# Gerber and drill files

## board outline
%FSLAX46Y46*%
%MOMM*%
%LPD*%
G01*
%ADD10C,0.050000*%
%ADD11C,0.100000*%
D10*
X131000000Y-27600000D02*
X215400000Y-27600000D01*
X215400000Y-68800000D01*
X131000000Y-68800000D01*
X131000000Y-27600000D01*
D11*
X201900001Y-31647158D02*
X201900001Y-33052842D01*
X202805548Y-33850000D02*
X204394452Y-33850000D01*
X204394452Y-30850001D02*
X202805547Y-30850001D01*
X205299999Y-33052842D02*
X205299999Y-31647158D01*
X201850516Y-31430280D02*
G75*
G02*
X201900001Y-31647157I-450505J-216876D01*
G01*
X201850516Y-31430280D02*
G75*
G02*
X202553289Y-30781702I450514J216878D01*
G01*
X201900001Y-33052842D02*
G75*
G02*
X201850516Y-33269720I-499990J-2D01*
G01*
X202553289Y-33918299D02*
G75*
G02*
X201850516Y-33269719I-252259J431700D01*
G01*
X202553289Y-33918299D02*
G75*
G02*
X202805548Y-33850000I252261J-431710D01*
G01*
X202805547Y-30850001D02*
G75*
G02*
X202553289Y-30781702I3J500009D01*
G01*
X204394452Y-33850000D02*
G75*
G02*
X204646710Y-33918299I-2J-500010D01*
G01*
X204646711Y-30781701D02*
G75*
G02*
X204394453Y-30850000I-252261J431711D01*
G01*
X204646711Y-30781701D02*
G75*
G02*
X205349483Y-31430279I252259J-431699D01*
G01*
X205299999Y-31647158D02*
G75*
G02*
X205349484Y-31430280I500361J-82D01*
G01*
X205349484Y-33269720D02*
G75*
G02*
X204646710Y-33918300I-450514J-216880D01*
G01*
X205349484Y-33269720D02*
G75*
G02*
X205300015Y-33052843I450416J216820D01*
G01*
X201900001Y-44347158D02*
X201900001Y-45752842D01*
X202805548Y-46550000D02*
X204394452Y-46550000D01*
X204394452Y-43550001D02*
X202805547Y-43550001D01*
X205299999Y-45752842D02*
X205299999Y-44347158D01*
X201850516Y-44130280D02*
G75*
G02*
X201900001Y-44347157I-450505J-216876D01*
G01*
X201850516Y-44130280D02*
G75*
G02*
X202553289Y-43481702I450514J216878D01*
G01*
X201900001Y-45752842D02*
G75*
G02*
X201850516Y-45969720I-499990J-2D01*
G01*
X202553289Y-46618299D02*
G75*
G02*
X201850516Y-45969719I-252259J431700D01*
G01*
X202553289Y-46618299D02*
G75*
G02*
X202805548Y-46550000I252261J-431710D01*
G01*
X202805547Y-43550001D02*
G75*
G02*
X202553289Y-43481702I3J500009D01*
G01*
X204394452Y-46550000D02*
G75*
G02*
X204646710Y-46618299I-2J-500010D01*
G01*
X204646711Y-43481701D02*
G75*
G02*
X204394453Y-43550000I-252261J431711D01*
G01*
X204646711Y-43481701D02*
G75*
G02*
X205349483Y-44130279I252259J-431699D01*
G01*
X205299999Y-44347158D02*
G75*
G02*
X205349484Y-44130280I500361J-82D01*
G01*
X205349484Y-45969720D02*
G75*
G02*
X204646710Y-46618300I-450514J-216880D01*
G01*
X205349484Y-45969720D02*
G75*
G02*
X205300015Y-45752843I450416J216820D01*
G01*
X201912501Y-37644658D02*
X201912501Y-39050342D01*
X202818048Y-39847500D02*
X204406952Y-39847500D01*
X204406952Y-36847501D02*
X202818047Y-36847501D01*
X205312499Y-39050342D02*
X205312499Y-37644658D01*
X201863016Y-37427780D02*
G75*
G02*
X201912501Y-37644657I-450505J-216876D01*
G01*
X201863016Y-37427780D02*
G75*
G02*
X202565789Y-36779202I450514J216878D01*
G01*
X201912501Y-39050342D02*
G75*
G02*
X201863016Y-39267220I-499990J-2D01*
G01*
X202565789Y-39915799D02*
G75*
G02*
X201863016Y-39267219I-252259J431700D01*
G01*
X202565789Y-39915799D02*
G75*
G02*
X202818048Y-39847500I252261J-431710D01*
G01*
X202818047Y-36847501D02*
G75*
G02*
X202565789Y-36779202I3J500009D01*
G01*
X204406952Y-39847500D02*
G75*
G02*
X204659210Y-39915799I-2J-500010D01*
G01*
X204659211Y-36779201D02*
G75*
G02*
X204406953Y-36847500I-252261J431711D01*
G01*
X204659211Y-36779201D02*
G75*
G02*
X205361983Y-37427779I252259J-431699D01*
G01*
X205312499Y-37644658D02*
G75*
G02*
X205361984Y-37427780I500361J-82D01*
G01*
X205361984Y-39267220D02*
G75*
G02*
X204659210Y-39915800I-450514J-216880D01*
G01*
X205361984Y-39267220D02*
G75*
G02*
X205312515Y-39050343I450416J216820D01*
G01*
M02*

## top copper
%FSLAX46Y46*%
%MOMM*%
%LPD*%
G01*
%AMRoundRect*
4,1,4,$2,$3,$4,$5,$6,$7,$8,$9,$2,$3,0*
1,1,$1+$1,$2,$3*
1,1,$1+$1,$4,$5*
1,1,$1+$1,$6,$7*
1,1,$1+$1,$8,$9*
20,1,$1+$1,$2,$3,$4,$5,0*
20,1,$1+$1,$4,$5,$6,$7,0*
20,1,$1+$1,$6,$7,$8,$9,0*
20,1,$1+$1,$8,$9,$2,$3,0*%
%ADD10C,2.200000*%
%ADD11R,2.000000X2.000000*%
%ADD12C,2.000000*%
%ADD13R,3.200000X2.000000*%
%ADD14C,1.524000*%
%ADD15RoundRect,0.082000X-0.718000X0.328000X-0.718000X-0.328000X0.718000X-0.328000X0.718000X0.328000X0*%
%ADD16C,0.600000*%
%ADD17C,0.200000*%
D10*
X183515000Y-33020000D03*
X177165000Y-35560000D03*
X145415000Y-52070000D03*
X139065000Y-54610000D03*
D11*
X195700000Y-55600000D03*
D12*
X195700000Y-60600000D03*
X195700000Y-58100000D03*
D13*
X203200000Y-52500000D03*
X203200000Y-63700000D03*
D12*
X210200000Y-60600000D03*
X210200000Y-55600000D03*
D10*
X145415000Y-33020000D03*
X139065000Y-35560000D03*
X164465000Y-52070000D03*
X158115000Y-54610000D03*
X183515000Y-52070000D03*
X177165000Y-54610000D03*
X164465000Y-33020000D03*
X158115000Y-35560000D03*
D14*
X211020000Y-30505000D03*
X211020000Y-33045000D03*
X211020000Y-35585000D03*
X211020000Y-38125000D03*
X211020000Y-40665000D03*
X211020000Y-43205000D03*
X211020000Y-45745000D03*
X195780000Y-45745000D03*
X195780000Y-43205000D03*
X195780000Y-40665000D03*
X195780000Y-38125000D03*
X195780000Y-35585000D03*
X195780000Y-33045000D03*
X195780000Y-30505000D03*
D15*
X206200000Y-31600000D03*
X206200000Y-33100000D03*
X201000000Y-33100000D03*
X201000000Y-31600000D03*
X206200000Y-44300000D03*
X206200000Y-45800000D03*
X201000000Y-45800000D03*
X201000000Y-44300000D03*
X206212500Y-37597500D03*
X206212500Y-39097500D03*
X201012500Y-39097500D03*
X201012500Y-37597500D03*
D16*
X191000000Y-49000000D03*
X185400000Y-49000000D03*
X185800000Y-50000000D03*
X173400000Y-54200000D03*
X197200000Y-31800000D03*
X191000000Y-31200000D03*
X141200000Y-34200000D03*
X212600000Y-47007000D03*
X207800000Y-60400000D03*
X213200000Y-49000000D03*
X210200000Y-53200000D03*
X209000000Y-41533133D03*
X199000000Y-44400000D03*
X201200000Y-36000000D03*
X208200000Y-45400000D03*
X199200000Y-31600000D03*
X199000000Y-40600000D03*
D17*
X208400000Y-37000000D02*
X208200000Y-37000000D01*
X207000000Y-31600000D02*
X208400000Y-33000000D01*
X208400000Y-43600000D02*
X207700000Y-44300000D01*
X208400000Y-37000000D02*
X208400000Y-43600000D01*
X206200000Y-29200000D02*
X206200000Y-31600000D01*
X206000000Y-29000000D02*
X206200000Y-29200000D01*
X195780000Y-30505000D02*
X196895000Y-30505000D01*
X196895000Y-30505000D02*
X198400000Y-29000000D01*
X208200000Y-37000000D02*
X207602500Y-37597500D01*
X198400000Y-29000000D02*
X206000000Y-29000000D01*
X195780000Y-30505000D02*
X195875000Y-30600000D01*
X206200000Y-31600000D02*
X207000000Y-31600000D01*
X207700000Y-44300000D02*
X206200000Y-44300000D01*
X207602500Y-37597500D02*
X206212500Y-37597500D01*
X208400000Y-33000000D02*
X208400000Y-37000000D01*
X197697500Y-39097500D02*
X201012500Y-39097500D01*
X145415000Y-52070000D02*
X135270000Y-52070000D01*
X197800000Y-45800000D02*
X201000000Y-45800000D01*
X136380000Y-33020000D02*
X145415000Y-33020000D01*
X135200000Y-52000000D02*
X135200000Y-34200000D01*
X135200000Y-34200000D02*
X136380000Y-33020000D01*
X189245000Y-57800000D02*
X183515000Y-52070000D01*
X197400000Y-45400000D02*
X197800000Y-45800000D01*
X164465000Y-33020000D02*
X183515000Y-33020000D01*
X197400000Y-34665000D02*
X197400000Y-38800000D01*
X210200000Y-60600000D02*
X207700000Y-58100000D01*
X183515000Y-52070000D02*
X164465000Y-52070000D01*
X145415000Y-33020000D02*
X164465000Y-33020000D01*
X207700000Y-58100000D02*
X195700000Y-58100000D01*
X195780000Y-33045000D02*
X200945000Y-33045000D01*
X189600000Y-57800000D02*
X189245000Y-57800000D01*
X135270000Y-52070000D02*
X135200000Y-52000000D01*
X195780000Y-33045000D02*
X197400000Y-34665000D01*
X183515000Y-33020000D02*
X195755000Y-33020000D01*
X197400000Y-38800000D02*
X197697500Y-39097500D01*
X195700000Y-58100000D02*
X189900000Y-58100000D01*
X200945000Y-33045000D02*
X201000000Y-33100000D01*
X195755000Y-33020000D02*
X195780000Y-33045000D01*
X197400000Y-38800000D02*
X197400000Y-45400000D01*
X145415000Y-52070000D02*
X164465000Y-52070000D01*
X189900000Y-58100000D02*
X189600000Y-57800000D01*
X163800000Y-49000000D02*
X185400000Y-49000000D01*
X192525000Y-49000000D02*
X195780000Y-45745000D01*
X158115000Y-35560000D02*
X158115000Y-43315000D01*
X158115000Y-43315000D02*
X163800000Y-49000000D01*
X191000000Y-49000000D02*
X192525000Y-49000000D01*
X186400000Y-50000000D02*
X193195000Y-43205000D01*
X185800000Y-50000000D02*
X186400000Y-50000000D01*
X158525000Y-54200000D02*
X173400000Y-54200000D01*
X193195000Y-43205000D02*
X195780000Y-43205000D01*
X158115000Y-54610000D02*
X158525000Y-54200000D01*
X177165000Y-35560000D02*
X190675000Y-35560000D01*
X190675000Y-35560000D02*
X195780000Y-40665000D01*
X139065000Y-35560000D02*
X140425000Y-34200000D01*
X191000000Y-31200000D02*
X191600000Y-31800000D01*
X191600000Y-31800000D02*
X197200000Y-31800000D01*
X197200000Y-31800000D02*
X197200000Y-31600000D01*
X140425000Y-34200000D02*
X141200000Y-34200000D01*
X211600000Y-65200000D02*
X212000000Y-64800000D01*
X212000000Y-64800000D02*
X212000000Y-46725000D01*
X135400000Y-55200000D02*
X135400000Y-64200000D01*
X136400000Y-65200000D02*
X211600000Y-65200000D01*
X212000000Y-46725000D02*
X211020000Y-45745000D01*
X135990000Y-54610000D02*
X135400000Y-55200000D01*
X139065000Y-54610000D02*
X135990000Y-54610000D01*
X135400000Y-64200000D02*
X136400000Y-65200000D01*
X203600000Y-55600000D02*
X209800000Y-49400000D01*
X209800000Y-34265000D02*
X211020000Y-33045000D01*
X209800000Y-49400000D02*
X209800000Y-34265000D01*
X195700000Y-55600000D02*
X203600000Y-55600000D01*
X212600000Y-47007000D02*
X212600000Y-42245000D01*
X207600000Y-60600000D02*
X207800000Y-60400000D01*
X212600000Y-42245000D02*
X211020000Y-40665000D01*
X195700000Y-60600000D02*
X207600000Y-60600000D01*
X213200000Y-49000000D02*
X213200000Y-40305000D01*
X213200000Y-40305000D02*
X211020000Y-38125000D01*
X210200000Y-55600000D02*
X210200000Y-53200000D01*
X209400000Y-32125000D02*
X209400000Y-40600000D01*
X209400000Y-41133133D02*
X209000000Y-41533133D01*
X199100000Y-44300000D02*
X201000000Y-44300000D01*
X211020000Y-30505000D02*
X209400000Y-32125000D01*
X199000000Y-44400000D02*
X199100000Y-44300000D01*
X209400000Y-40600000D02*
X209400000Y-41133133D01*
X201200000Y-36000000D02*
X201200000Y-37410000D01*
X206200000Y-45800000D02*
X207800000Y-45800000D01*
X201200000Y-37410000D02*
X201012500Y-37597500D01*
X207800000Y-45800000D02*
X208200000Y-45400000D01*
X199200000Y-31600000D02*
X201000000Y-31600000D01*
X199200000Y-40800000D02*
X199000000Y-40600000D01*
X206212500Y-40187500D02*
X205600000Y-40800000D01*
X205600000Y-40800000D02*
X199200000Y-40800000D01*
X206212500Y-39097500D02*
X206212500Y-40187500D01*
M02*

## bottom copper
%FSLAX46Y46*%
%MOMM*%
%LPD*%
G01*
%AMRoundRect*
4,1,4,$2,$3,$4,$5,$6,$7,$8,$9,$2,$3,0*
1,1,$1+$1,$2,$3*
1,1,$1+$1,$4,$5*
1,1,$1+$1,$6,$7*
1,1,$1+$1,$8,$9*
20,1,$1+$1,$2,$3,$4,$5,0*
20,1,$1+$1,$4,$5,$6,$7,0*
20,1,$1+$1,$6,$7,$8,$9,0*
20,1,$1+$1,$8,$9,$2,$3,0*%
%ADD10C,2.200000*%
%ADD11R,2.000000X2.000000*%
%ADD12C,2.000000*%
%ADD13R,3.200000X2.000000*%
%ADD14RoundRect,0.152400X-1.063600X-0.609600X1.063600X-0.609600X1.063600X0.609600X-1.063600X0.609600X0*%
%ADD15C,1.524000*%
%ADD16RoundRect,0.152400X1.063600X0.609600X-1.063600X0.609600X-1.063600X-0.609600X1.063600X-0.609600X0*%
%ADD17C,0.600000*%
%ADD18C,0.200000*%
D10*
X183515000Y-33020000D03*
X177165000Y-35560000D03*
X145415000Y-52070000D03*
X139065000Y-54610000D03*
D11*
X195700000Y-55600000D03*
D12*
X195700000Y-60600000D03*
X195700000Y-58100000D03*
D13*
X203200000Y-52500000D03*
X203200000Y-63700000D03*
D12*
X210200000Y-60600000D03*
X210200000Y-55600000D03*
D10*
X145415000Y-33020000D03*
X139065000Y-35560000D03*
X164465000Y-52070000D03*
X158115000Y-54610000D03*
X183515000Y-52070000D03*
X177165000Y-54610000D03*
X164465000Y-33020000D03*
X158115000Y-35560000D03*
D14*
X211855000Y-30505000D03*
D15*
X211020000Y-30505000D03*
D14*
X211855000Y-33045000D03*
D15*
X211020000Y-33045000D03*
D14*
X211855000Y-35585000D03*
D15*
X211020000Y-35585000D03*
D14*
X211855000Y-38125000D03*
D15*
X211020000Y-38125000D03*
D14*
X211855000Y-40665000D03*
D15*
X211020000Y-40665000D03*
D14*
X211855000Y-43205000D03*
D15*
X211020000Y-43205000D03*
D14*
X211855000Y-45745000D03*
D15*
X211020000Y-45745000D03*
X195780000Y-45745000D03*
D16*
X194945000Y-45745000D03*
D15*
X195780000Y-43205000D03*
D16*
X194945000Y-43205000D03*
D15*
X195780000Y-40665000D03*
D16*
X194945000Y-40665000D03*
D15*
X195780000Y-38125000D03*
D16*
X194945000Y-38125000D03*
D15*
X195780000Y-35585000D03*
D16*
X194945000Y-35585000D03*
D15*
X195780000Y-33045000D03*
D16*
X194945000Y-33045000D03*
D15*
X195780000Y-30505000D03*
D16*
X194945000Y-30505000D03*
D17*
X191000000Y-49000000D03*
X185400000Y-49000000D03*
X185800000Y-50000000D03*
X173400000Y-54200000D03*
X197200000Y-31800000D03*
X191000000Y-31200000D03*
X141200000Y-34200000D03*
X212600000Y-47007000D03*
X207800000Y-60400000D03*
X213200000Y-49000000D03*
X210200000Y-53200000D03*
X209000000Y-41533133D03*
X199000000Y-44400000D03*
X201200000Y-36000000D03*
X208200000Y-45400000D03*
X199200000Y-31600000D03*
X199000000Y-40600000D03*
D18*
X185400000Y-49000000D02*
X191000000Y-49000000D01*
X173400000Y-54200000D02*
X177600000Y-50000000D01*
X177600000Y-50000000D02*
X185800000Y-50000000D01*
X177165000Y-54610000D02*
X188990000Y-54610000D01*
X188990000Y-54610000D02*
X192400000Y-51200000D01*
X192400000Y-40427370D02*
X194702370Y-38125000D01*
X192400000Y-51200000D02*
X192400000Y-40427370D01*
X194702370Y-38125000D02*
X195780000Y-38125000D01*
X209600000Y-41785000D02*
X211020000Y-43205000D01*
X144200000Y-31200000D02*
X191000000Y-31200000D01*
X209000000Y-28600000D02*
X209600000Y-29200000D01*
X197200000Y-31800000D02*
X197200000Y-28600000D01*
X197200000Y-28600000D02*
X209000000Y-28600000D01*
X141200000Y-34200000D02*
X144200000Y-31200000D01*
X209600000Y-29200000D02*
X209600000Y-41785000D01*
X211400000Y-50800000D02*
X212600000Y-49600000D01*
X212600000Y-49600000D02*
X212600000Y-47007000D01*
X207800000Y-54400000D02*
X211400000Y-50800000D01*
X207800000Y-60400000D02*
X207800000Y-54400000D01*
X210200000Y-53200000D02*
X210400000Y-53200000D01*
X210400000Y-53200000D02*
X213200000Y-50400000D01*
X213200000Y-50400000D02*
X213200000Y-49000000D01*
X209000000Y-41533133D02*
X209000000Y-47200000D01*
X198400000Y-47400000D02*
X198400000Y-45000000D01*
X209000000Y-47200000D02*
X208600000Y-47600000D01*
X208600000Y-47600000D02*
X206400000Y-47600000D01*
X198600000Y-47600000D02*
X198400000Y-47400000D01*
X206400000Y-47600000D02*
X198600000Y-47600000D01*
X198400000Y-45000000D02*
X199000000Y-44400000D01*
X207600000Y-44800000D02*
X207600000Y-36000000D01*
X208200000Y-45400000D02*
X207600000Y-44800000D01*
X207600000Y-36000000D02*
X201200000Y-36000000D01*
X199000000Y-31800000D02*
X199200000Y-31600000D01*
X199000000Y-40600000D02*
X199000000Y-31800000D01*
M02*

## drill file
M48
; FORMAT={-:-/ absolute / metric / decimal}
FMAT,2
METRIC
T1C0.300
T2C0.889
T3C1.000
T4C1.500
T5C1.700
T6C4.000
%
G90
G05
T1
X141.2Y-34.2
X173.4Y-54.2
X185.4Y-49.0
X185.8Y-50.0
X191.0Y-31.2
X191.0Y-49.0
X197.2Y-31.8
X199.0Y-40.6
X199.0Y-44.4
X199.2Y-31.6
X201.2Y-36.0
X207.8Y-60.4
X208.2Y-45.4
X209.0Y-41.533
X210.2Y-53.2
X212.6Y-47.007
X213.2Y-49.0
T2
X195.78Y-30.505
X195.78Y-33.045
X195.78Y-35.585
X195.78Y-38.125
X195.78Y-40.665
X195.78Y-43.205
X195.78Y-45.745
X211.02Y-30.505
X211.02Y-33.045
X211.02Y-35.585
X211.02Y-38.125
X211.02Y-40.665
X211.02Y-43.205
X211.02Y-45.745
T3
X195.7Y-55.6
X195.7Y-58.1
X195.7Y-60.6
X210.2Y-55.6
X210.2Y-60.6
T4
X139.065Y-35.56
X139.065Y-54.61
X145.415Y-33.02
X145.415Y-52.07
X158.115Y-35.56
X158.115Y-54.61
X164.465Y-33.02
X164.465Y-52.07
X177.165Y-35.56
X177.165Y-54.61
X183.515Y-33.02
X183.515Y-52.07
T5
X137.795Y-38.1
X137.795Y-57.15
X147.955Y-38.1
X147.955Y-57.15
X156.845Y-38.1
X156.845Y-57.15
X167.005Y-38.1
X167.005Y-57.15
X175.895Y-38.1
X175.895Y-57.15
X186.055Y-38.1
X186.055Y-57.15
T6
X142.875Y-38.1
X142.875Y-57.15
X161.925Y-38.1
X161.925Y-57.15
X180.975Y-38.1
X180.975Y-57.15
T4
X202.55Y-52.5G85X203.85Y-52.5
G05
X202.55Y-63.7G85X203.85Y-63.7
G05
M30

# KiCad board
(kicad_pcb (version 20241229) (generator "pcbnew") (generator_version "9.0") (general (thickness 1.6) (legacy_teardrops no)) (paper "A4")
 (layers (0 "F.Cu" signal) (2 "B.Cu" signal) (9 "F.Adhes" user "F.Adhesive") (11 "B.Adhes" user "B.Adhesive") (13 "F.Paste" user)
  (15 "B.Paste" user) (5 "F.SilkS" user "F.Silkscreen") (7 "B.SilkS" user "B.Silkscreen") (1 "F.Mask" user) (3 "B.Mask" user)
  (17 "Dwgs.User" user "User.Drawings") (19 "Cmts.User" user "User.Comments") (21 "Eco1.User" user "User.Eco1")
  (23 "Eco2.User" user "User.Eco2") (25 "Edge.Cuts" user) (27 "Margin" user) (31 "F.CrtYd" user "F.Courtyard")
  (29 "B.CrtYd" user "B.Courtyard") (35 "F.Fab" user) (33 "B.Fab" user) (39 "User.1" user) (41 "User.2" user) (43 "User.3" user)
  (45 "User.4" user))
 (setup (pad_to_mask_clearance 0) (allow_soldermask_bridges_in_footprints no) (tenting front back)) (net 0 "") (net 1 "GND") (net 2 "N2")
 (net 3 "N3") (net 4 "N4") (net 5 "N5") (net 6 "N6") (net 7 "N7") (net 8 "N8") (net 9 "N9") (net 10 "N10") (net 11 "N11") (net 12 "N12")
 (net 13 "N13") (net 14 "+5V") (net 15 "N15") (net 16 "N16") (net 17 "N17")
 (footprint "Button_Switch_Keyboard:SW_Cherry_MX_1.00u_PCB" (layer "F.Cu") (at 183.515 33.02)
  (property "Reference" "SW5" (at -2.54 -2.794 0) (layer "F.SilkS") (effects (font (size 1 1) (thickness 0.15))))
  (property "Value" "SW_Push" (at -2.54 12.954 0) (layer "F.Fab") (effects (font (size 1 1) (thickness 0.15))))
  (pad "" np_thru_hole circle (at -7.62 5.08) (size 1.7 1.7) (drill 1.7) (layers "*.Cu" "*.Mask"))
  (pad "" np_thru_hole circle (at -2.54 5.08) (size 4 4) (drill 4) (layers "*.Cu" "*.Mask"))
  (pad "" np_thru_hole circle (at 2.54 5.08) (size 1.7 1.7) (drill 1.7) (layers "*.Cu" "*.Mask"))
  (pad "1" thru_hole circle (at 0 0) (size 2.2 2.2) (drill 1.5) (layers "*.Cu" "*.Mask") (remove_unused_layers no) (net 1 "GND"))
  (pad "2" thru_hole circle (at -6.35 2.54) (size 2.2 2.2) (drill 1.5) (layers "*.Cu" "*.Mask") (remove_unused_layers no) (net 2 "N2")))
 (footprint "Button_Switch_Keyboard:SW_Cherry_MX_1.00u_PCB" (layer "F.Cu") (at 145.415 52.07)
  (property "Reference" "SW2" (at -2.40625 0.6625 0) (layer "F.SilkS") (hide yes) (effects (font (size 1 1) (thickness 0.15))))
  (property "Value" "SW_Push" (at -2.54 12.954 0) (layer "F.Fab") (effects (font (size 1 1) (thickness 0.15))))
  (pad "" np_thru_hole circle (at -7.62 5.08) (size 1.7 1.7) (drill 1.7) (layers "*.Cu" "*.Mask"))
  (pad "" np_thru_hole circle (at -2.54 5.08) (size 4 4) (drill 4) (layers "*.Cu" "*.Mask"))
  (pad "" np_thru_hole circle (at 2.54 5.08) (size 1.7 1.7) (drill 1.7) (layers "*.Cu" "*.Mask"))
  (pad "1" thru_hole circle (at 0 0) (size 2.2 2.2) (drill 1.5) (layers "*.Cu" "*.Mask") (remove_unused_layers no) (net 1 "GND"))
  (pad "2" thru_hole circle (at -6.35 2.54) (size 2.2 2.2) (drill 1.5) (layers "*.Cu" "*.Mask") (remove_unused_layers no) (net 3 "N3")))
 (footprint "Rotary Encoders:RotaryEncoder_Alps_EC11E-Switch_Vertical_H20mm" (layer "F.Cu") (at 195.7 55.6)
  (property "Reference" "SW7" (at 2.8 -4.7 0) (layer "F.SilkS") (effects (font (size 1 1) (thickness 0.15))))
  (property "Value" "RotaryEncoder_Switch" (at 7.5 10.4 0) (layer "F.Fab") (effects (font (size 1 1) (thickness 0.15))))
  (pad "A" thru_hole rect (at 0 0) (size 2 2) (drill 1) (layers "*.Cu" "*.Mask") (remove_unused_layers no) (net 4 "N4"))
  (pad "B" thru_hole circle (at 0 5) (size 2 2) (drill 1) (layers "*.Cu" "*.Mask") (remove_unused_layers no) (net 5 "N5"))
  (pad "C" thru_hole circle (at 0 2.5) (size 2 2) (drill 1) (layers "*.Cu" "*.Mask") (remove_unused_layers no) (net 1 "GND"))
  (pad "MP" thru_hole rect (at 7.5 -3.1) (size 3.2 2) (drill oval 2.8 1.5) (layers "*.Cu" "*.Mask") (remove_unused_layers no))
  (pad "MP" thru_hole rect (at 7.5 8.1) (size 3.2 2) (drill oval 2.8 1.5) (layers "*.Cu" "*.Mask") (remove_unused_layers no))
  (pad "S1" thru_hole circle (at 14.5 5) (size 2 2) (drill 1) (layers "*.Cu" "*.Mask") (remove_unused_layers no) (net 1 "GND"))
  (pad "S2" thru_hole circle (at 14.5 0) (size 2 2) (drill 1) (layers "*.Cu" "*.Mask") (remove_unused_layers no) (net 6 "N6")))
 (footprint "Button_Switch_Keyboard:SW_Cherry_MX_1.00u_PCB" (layer "F.Cu") (at 145.415 33.02)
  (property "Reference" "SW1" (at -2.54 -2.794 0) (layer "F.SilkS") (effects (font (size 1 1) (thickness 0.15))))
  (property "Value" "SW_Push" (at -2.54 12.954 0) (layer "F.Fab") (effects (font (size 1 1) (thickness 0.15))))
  (pad "" np_thru_hole circle (at -7.62 5.08) (size 1.7 1.7) (drill 1.7) (layers "*.Cu" "*.Mask"))
  (pad "" np_thru_hole circle (at -2.54 5.08) (size 4 4) (drill 4) (layers "*.Cu" "*.Mask"))
  (pad "" np_thru_hole circle (at 2.54 5.08) (size 1.7 1.7) (drill 1.7) (layers "*.Cu" "*.Mask"))
  (pad "1" thru_hole circle (at 0 0) (size 2.2 2.2) (drill 1.5) (layers "*.Cu" "*.Mask") (remove_unused_layers no) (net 1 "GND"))
  (pad "2" thru_hole circle (at -6.35 2.54) (size 2.2 2.2) (drill 1.5) (layers "*.Cu" "*.Mask") (remove_unused_layers no) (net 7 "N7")))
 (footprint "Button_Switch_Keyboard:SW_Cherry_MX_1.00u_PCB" (layer "F.Cu") (at 164.465 52.07)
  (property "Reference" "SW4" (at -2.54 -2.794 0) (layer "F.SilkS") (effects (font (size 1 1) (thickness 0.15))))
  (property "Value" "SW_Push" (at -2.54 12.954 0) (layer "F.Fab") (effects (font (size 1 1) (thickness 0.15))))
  (pad "" np_thru_hole circle (at -7.62 5.08) (size 1.7 1.7) (drill 1.7) (layers "*.Cu" "*.Mask"))
  (pad "" np_thru_hole circle (at -2.54 5.08) (size 4 4) (drill 4) (layers "*.Cu" "*.Mask"))
  (pad "" np_thru_hole circle (at 2.54 5.08) (size 1.7 1.7) (drill 1.7) (layers "*.Cu" "*.Mask"))
  (pad "1" thru_hole circle (at 0 0) (size 2.2 2.2) (drill 1.5) (layers "*.Cu" "*.Mask") (remove_unused_layers no) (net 1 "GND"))
  (pad "2" thru_hole circle (at -6.35 2.54) (size 2.2 2.2) (drill 1.5) (layers "*.Cu" "*.Mask") (remove_unused_layers no) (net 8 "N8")))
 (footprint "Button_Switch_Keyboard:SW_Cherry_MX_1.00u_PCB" (layer "F.Cu") (at 183.515 52.07)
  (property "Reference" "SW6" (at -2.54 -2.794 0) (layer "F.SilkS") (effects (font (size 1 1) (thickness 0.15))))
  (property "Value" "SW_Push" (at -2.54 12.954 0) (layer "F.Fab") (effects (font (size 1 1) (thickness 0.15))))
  (pad "" np_thru_hole circle (at -7.62 5.08) (size 1.7 1.7) (drill 1.7) (layers "*.Cu" "*.Mask"))
  (pad "" np_thru_hole circle (at -2.54 5.08) (size 4 4) (drill 4) (layers "*.Cu" "*.Mask"))
  (pad "" np_thru_hole circle (at 2.54 5.08) (size 1.7 1.7) (drill 1.7) (layers "*.Cu" "*.Mask"))
  (pad "1" thru_hole circle (at 0 0) (size 2.2 2.2) (drill 1.5) (layers "*.Cu" "*.Mask") (remove_unused_layers no) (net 1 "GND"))
  (pad "2" thru_hole circle (at -6.35 2.54) (size 2.2 2.2) (drill 1.5) (layers "*.Cu" "*.Mask") (remove_unused_layers no) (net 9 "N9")))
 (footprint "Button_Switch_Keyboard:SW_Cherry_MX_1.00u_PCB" (layer "F.Cu") (at 164.465 33.02)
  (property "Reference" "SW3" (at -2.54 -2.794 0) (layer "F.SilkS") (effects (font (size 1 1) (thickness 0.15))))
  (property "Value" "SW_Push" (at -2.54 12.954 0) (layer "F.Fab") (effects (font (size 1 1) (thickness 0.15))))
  (pad "" np_thru_hole circle (at -7.62 5.08) (size 1.7 1.7) (drill 1.7) (layers "*.Cu" "*.Mask"))
  (pad "" np_thru_hole circle (at -2.54 5.08) (size 4 4) (drill 4) (layers "*.Cu" "*.Mask"))
  (pad "" np_thru_hole circle (at 2.54 5.08) (size 1.7 1.7) (drill 1.7) (layers "*.Cu" "*.Mask"))
  (pad "1" thru_hole circle (at 0 0) (size 2.2 2.2) (drill 1.5) (layers "*.Cu" "*.Mask") (remove_unused_layers no) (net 1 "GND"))
  (pad "2" thru_hole circle (at -6.35 2.54) (size 2.2 2.2) (drill 1.5) (layers "*.Cu" "*.Mask") (remove_unused_layers no) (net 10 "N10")))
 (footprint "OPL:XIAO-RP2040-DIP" (layer "B.Cu") (at 203.4 38.125 180)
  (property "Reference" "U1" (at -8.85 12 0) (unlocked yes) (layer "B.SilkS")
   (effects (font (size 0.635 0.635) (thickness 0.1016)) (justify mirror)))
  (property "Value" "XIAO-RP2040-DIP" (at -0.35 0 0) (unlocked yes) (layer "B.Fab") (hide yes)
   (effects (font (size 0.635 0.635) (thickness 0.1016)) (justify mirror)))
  (pad "1" smd roundrect (at -8.455 7.62) (size 2.432 1.524) (layers "B.Cu" "B.Mask") (roundrect_rratio 0.1) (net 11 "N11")
   (thermal_bridge_angle 45))
  (pad "1" thru_hole circle (at -7.62 7.62) (size 1.524 1.524) (drill 0.889) (layers "*.Cu" "*.Mask") (remove_unused_layers no)
   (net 11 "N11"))
  (pad "2" smd roundrect (at -8.455 5.08) (size 2.432 1.524) (layers "B.Cu" "B.Mask") (roundrect_rratio 0.1) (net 4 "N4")
   (thermal_bridge_angle 45))
  (pad "2" thru_hole circle (at -7.62 5.08) (size 1.524 1.524) (drill 0.889) (layers "*.Cu" "*.Mask") (remove_unused_layers no) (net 4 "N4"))
  (pad "3" smd roundrect (at -8.455 2.54) (size 2.432 1.524) (layers "B.Cu" "B.Mask") (roundrect_rratio 0.1) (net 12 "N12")
   (thermal_bridge_angle 45))
  (pad "3" thru_hole circle (at -7.62 2.54) (size 1.524 1.524) (drill 0.889) (layers "*.Cu" "*.Mask") (remove_unused_layers no)
   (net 12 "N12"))
  (pad "4" smd roundrect (at -8.455 0) (size 2.432 1.524) (layers "B.Cu" "B.Mask") (roundrect_rratio 0.1) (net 6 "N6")
   (thermal_bridge_angle 45))
  (pad "4" thru_hole circle (at -7.62 0) (size 1.524 1.524) (drill 0.889) (layers "*.Cu" "*.Mask") (remove_unused_layers no) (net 6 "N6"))
  (pad "5" smd roundrect (at -8.455 -2.54) (size 2.432 1.524) (layers "B.Cu" "B.Mask") (roundrect_rratio 0.1) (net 5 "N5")
   (thermal_bridge_angle 45))
  (pad "5" thru_hole circle (at -7.62 -2.54) (size 1.524 1.524) (drill 0.889) (layers "*.Cu" "*.Mask") (remove_unused_layers no)
   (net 5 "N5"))
  (pad "6" smd roundrect (at -8.455 -5.08) (size 2.432 1.524) (layers "B.Cu" "B.Mask") (roundrect_rratio 0.1) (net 7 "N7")
   (thermal_bridge_angle 45))
  (pad "6" thru_hole circle (at -7.62 -5.08) (size 1.524 1.524) (drill 0.889) (layers "*.Cu" "*.Mask") (remove_unused_layers no)
   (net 7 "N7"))
  (pad "7" smd roundrect (at -8.455 -7.62) (size 2.432 1.524) (layers "B.Cu" "B.Mask") (roundrect_rratio 0.1) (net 3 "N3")
   (thermal_bridge_angle 45))
  (pad "7" thru_hole circle (at -7.62 -7.62) (size 1.524 1.524) (drill 0.889) (layers "*.Cu" "*.Mask") (remove_unused_layers no)
   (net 3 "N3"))
  (pad "8" thru_hole circle (at 7.62 -7.62 180) (size 1.524 1.524) (drill 0.889) (layers "*.Cu" "*.Mask") (remove_unused_layers no)
   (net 10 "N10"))
  (pad "8" smd roundrect (at 8.455 -7.62 180) (size 2.432 1.524) (layers "B.Cu" "B.Mask") (roundrect_rratio 0.1) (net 10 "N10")
   (thermal_bridge_angle 45))
  (pad "9" thru_hole circle (at 7.62 -5.08 180) (size 1.524 1.524) (drill 0.889) (layers "*.Cu" "*.Mask") (remove_unused_layers no)
   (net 8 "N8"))
  (pad "9" smd roundrect (at 8.455 -5.08 180) (size 2.432 1.524) (layers "B.Cu" "B.Mask") (roundrect_rratio 0.1) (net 8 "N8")
   (thermal_bridge_angle 45))
  (pad "10" thru_hole circle (at 7.62 -2.54 180) (size 1.524 1.524) (drill 0.889) (layers "*.Cu" "*.Mask") (remove_unused_layers no)
   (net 2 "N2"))
  (pad "10" smd roundrect (at 8.455 -2.54 180) (size 2.432 1.524) (layers "B.Cu" "B.Mask") (roundrect_rratio 0.1) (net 2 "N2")
   (thermal_bridge_angle 45))
  (pad "11" thru_hole circle (at 7.62 0 180) (size 1.524 1.524) (drill 0.889) (layers "*.Cu" "*.Mask") (remove_unused_layers no)
   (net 9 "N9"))
  (pad "11" smd roundrect (at 8.455 0 180) (size 2.432 1.524) (layers "B.Cu" "B.Mask") (roundrect_rratio 0.1) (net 9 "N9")
   (thermal_bridge_angle 45))
  (pad "12" thru_hole circle (at 7.62 2.54 180) (size 1.524 1.524) (drill 0.889) (layers "*.Cu" "*.Mask") (remove_unused_layers no)
   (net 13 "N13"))
  (pad "12" smd roundrect (at 8.455 2.54 180) (size 2.432 1.524) (layers "B.Cu" "B.Mask") (roundrect_rratio 0.1) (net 13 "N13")
   (thermal_bridge_angle 45))
  (pad "13" thru_hole circle (at 7.62 5.08 180) (size 1.524 1.524) (drill 0.889) (layers "*.Cu" "*.Mask") (remove_unused_layers no)
   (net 1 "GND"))
  (pad "13" smd roundrect (at 8.455 5.08 180) (size 2.432 1.524) (layers "B.Cu" "B.Mask") (roundrect_rratio 0.1) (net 1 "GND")
   (thermal_bridge_angle 45))
  (pad "14" thru_hole circle (at 7.62 7.62 180) (size 1.524 1.524) (drill 0.889) (layers "*.Cu" "*.Mask") (remove_unused_layers no)
   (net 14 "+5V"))
  (pad "14" smd roundrect (at 8.455 7.62 180) (size 2.432 1.524) (layers "B.Cu" "B.Mask") (roundrect_rratio 0.1) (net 14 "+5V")
   (thermal_bridge_angle 45)))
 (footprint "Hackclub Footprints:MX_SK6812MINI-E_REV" (layer "B.Cu") (at 203.6 37.43)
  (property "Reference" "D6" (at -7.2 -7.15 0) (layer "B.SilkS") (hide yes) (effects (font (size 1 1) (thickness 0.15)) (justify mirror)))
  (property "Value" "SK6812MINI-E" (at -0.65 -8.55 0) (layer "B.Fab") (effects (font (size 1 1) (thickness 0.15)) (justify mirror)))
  (fp_line (start -1.699999 -5.782842) (end -1.699999 -4.377158) (stroke (width 0.1) (type solid)) (layer "Edge.Cuts"))
  (fp_line (start -0.794452 -3.58) (end 0.794452 -3.58) (stroke (width 0.1) (type solid)) (layer "Edge.Cuts"))
  (fp_line (start 0.794452 -6.579999) (end -0.794453 -6.579999) (stroke (width 0.1) (type solid)) (layer "Edge.Cuts"))
  (fp_line (start 1.699999 -4.377158) (end 1.699999 -5.782842) (stroke (width 0.1) (type solid)) (layer "Edge.Cuts"))
  (fp_arc (start -1.749484 -5.99972) (mid -1.712527 -5.894068) (end -1.699999 -5.782843) (stroke (width 0.1) (type solid))
   (layer "Edge.Cuts"))
  (fp_arc (start -1.749484 -5.99972) (mid -1.638071 -6.584035) (end -1.046711 -6.648298) (stroke (width 0.1) (type solid))
   (layer "Edge.Cuts"))
  (fp_arc (start -1.699999 -4.377158) (mid -1.712527 -4.265932) (end -1.749484 -4.16028) (stroke (width 0.1) (type solid))
   (layer "Edge.Cuts"))
  (fp_arc (start -1.046711 -3.511701) (mid -1.638072 -3.575965) (end -1.749484 -4.160281) (stroke (width 0.1) (type solid))
   (layer "Edge.Cuts"))
  (fp_arc (start -1.046711 -3.511701) (mid -0.925123 -3.562623) (end -0.794452 -3.58) (stroke (width 0.1) (type solid)) (layer "Edge.Cuts"))
  (fp_arc (start -0.794453 -6.579999) (mid -0.925123 -6.597376) (end -1.046711 -6.648298) (stroke (width 0.1) (type solid))
   (layer "Edge.Cuts"))
  (fp_arc (start 0.794452 -3.58) (mid 0.925122 -3.562623) (end 1.04671 -3.511701) (stroke (width 0.1) (type solid)) (layer "Edge.Cuts"))
  (fp_arc (start 1.046711 -6.648299) (mid 0.925123 -6.597377) (end 0.794453 -6.58) (stroke (width 0.1) (type solid)) (layer "Edge.Cuts"))
  (fp_arc (start 1.046711 -6.648299) (mid 1.638071 -6.584036) (end 1.749484 -5.99972) (stroke (width 0.1) (type solid)) (layer "Edge.Cuts"))
  (fp_arc (start 1.699999 -5.782842) (mid 1.712536 -5.894065) (end 1.749484 -5.99972) (stroke (width 0.1) (type solid)) (layer "Edge.Cuts"))
  (fp_arc (start 1.749484 -4.16028) (mid 1.638072 -3.575963) (end 1.046711 -3.511703) (stroke (width 0.1) (type solid)) (layer "Edge.Cuts"))
  (fp_arc (start 1.749484 -4.16028) (mid 1.712526 -4.265931) (end 1.699999 -4.377157) (stroke (width 0.1) (type solid)) (layer "Edge.Cuts"))
  (pad "1" smd roundrect (at 2.6 -5.83 270) (size 0.82 1.6) (layers "F.Cu" "F.Mask" "F.Paste") (roundrect_rratio 0.1) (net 14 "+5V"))
  (pad "2" smd roundrect (at 2.6 -4.33 270) (size 0.82 1.6) (layers "F.Cu" "F.Mask" "F.Paste") (roundrect_rratio 0.1) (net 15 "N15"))
  (pad "3" smd roundrect (at -2.6 -4.33 270) (size 0.82 1.6) (layers "F.Cu" "F.Mask" "F.Paste") (roundrect_rratio 0.1) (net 1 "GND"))
  (pad "4" smd roundrect (at -2.6 -5.83 270) (size 0.82 1.6) (layers "F.Cu" "F.Mask" "F.Paste") (roundrect_rratio 0.1) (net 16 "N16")))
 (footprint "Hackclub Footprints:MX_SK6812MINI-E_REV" (layer "B.Cu") (at 203.6 50.13)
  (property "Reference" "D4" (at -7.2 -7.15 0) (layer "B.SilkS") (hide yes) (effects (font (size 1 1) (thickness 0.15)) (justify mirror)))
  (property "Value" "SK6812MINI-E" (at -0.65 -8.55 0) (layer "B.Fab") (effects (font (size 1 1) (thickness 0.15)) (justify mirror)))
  (fp_line (start -1.699999 -5.782842) (end -1.699999 -4.377158) (stroke (width 0.1) (type solid)) (layer "Edge.Cuts"))
  (fp_line (start -0.794452 -3.58) (end 0.794452 -3.58) (stroke (width 0.1) (type solid)) (layer "Edge.Cuts"))
  (fp_line (start 0.794452 -6.579999) (end -0.794453 -6.579999) (stroke (width 0.1) (type solid)) (layer "Edge.Cuts"))
  (fp_line (start 1.699999 -4.377158) (end 1.699999 -5.782842) (stroke (width 0.1) (type solid)) (layer "Edge.Cuts"))
  (fp_arc (start -1.749484 -5.99972) (mid -1.712527 -5.894068) (end -1.699999 -5.782843) (stroke (width 0.1) (type solid))
   (layer "Edge.Cuts"))
  (fp_arc (start -1.749484 -5.99972) (mid -1.638071 -6.584035) (end -1.046711 -6.648298) (stroke (width 0.1) (type solid))
   (layer "Edge.Cuts"))
  (fp_arc (start -1.699999 -4.377158) (mid -1.712527 -4.265932) (end -1.749484 -4.16028) (stroke (width 0.1) (type solid))
   (layer "Edge.Cuts"))
  (fp_arc (start -1.046711 -3.511701) (mid -1.638072 -3.575965) (end -1.749484 -4.160281) (stroke (width 0.1) (type solid))
   (layer "Edge.Cuts"))
  (fp_arc (start -1.046711 -3.511701) (mid -0.925123 -3.562623) (end -0.794452 -3.58) (stroke (width 0.1) (type solid)) (layer "Edge.Cuts"))
  (fp_arc (start -0.794453 -6.579999) (mid -0.925123 -6.597376) (end -1.046711 -6.648298) (stroke (width 0.1) (type solid))
   (layer "Edge.Cuts"))
  (fp_arc (start 0.794452 -3.58) (mid 0.925122 -3.562623) (end 1.04671 -3.511701) (stroke (width 0.1) (type solid)) (layer "Edge.Cuts"))
  (fp_arc (start 1.046711 -6.648299) (mid 0.925123 -6.597377) (end 0.794453 -6.58) (stroke (width 0.1) (type solid)) (layer "Edge.Cuts"))
  (fp_arc (start 1.046711 -6.648299) (mid 1.638071 -6.584036) (end 1.749484 -5.99972) (stroke (width 0.1) (type solid)) (layer "Edge.Cuts"))
  (fp_arc (start 1.699999 -5.782842) (mid 1.712536 -5.894065) (end 1.749484 -5.99972) (stroke (width 0.1) (type solid)) (layer "Edge.Cuts"))
  (fp_arc (start 1.749484 -4.16028) (mid 1.638072 -3.575963) (end 1.046711 -3.511703) (stroke (width 0.1) (type solid)) (layer "Edge.Cuts"))
  (fp_arc (start 1.749484 -4.16028) (mid 1.712526 -4.265931) (end 1.699999 -4.377157) (stroke (width 0.1) (type solid)) (layer "Edge.Cuts"))
  (pad "1" smd roundrect (at 2.6 -5.83 270) (size 0.82 1.6) (layers "F.Cu" "F.Mask" "F.Paste") (roundrect_rratio 0.1) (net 14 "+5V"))
  (pad "2" smd roundrect (at 2.6 -4.33 270) (size 0.82 1.6) (layers "F.Cu" "F.Mask" "F.Paste") (roundrect_rratio 0.1) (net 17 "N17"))
  (pad "3" smd roundrect (at -2.6 -4.33 270) (size 0.82 1.6) (layers "F.Cu" "F.Mask" "F.Paste") (roundrect_rratio 0.1) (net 1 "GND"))
  (pad "4" smd roundrect (at -2.6 -5.83 270) (size 0.82 1.6) (layers "F.Cu" "F.Mask" "F.Paste") (roundrect_rratio 0.1) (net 11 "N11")))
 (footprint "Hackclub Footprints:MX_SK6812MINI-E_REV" (layer "B.Cu") (at 203.6125 43.4275)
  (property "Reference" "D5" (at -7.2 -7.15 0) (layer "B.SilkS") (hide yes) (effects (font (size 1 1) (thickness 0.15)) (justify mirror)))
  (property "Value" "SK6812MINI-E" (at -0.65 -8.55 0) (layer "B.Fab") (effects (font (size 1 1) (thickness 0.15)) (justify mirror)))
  (fp_line (start -1.699999 -5.782842) (end -1.699999 -4.377158) (stroke (width 0.1) (type solid)) (layer "Edge.Cuts"))
  (fp_line (start -0.794452 -3.58) (end 0.794452 -3.58) (stroke (width 0.1) (type solid)) (layer "Edge.Cuts"))
  (fp_line (start 0.794452 -6.579999) (end -0.794453 -6.579999) (stroke (width 0.1) (type solid)) (layer "Edge.Cuts"))
  (fp_line (start 1.699999 -4.377158) (end 1.699999 -5.782842) (stroke (width 0.1) (type solid)) (layer "Edge.Cuts"))
  (fp_arc (start -1.749484 -5.99972) (mid -1.712527 -5.894068) (end -1.699999 -5.782843) (stroke (width 0.1) (type solid))
   (layer "Edge.Cuts"))
  (fp_arc (start -1.749484 -5.99972) (mid -1.638071 -6.584035) (end -1.046711 -6.648298) (stroke (width 0.1) (type solid))
   (layer "Edge.Cuts"))
  (fp_arc (start -1.699999 -4.377158) (mid -1.712527 -4.265932) (end -1.749484 -4.16028) (stroke (width 0.1) (type solid))
   (layer "Edge.Cuts"))
  (fp_arc (start -1.046711 -3.511701) (mid -1.638072 -3.575965) (end -1.749484 -4.160281) (stroke (width 0.1) (type solid))
   (layer "Edge.Cuts"))
  (fp_arc (start -1.046711 -3.511701) (mid -0.925123 -3.562623) (end -0.794452 -3.58) (stroke (width 0.1) (type solid)) (layer "Edge.Cuts"))
  (fp_arc (start -0.794453 -6.579999) (mid -0.925123 -6.597376) (end -1.046711 -6.648298) (stroke (width 0.1) (type solid))
   (layer "Edge.Cuts"))
  (fp_arc (start 0.794452 -3.58) (mid 0.925122 -3.562623) (end 1.04671 -3.511701) (stroke (width 0.1) (type solid)) (layer "Edge.Cuts"))
  (fp_arc (start 1.046711 -6.648299) (mid 0.925123 -6.597377) (end 0.794453 -6.58) (stroke (width 0.1) (type solid)) (layer "Edge.Cuts"))
  (fp_arc (start 1.046711 -6.648299) (mid 1.638071 -6.584036) (end 1.749484 -5.99972) (stroke (width 0.1) (type solid)) (layer "Edge.Cuts"))
  (fp_arc (start 1.699999 -5.782842) (mid 1.712536 -5.894065) (end 1.749484 -5.99972) (stroke (width 0.1) (type solid)) (layer "Edge.Cuts"))
  (fp_arc (start 1.749484 -4.16028) (mid 1.638072 -3.575963) (end 1.046711 -3.511703) (stroke (width 0.1) (type solid)) (layer "Edge.Cuts"))
  (fp_arc (start 1.749484 -4.16028) (mid 1.712526 -4.265931) (end 1.699999 -4.377157) (stroke (width 0.1) (type solid)) (layer "Edge.Cuts"))
  (pad "1" smd roundrect (at 2.6 -5.83 270) (size 0.82 1.6) (layers "F.Cu" "F.Mask" "F.Paste") (roundrect_rratio 0.1) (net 14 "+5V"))
  (pad "2" smd roundrect (at 2.6 -4.33 270) (size 0.82 1.6) (layers "F.Cu" "F.Mask" "F.Paste") (roundrect_rratio 0.1) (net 16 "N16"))
  (pad "3" smd roundrect (at -2.6 -4.33 270) (size 0.82 1.6) (layers "F.Cu" "F.Mask" "F.Paste") (roundrect_rratio 0.1) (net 1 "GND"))
  (pad "4" smd roundrect (at -2.6 -5.83 270) (size 0.82 1.6) (layers "F.Cu" "F.Mask" "F.Paste") (roundrect_rratio 0.1) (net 17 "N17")))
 (gr_rect (start 131 27.6) (end 215.4 68.8) (stroke (width 0.05) (type default)) (fill no) (layer "Edge.Cuts"))
 (segment (start 208.4 37) (end 208.2 37) (width 0.2) (layer "F.Cu") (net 14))
 (segment (start 207 31.6) (end 208.4 33) (width 0.2) (layer "F.Cu") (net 14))
 (segment (start 208.4 43.6) (end 207.7 44.3) (width 0.2) (layer "F.Cu") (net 14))
 (segment (start 208.4 37) (end 208.4 43.6) (width 0.2) (layer "F.Cu") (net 14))
 (segment (start 206.2 29.2) (end 206.2 31.6) (width 0.2) (layer "F.Cu") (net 14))
 (segment (start 206 29) (end 206.2 29.2) (width 0.2) (layer "F.Cu") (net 14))
 (segment (start 195.78 30.505) (end 196.895 30.505) (width 0.2) (layer "F.Cu") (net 14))
 (segment (start 196.895 30.505) (end 198.4 29) (width 0.2) (layer "F.Cu") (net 14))
 (segment (start 208.2 37) (end 207.6025 37.5975) (width 0.2) (layer "F.Cu") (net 14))
 (segment (start 198.4 29) (end 206 29) (width 0.2) (layer "F.Cu") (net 14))
 (segment (start 195.78 30.505) (end 195.875 30.6) (width 0.2) (layer "F.Cu") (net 14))
 (segment (start 206.2 31.6) (end 207 31.6) (width 0.2) (layer "F.Cu") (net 14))
 (segment (start 207.7 44.3) (end 206.2 44.3) (width 0.2) (layer "F.Cu") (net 14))
 (segment (start 207.6025 37.5975) (end 206.2125 37.5975) (width 0.2) (layer "F.Cu") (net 14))
 (segment (start 208.4 33) (end 208.4 37) (width 0.2) (layer "F.Cu") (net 14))
 (segment (start 197.6975 39.0975) (end 201.0125 39.0975) (width 0.2) (layer "F.Cu") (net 1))
 (segment (start 145.415 52.07) (end 135.27 52.07) (width 0.2) (layer "F.Cu") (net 1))
 (segment (start 197.8 45.8) (end 201 45.8) (width 0.2) (layer "F.Cu") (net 1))
 (segment (start 136.38 33.02) (end 145.415 33.02) (width 0.2) (layer "F.Cu") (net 1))
 (segment (start 135.2 52) (end 135.2 34.2) (width 0.2) (layer "F.Cu") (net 1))
 (segment (start 135.2 34.2) (end 136.38 33.02) (width 0.2) (layer "F.Cu") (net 1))
 (segment (start 189.245 57.8) (end 183.515 52.07) (width 0.2) (layer "F.Cu") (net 1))
 (segment (start 197.4 45.4) (end 197.8 45.8) (width 0.2) (layer "F.Cu") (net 1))
 (segment (start 164.465 33.02) (end 183.515 33.02) (width 0.2) (layer "F.Cu") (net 1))
 (segment (start 197.4 34.665) (end 197.4 38.8) (width 0.2) (layer "F.Cu") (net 1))
 (segment (start 210.2 60.6) (end 207.7 58.1) (width 0.2) (layer "F.Cu") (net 1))
 (segment (start 183.515 52.07) (end 164.465 52.07) (width 0.2) (layer "F.Cu") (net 1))
 (segment (start 145.415 33.02) (end 164.465 33.02) (width 0.2) (layer "F.Cu") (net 1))
 (segment (start 207.7 58.1) (end 195.7 58.1) (width 0.2) (layer "F.Cu") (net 1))
 (segment (start 195.78 33.045) (end 200.945 33.045) (width 0.2) (layer "F.Cu") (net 1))
 (segment (start 189.6 57.8) (end 189.245 57.8) (width 0.2) (layer "F.Cu") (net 1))
 (segment (start 135.27 52.07) (end 135.2 52) (width 0.2) (layer "F.Cu") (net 1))
 (segment (start 195.78 33.045) (end 197.4 34.665) (width 0.2) (layer "F.Cu") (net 1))
 (segment (start 183.515 33.02) (end 195.755 33.02) (width 0.2) (layer "F.Cu") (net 1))
 (segment (start 197.4 38.8) (end 197.6975 39.0975) (width 0.2) (layer "F.Cu") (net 1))
 (segment (start 195.7 58.1) (end 189.9 58.1) (width 0.2) (layer "F.Cu") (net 1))
 (segment (start 200.945 33.045) (end 201 33.1) (width 0.2) (layer "F.Cu") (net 1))
 (segment (start 195.755 33.02) (end 195.78 33.045) (width 0.2) (layer "F.Cu") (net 1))
 (segment (start 197.4 38.8) (end 197.4 45.4) (width 0.2) (layer "F.Cu") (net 1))
 (segment (start 145.415 52.07) (end 164.465 52.07) (width 0.2) (layer "F.Cu") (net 1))
 (segment (start 189.9 58.1) (end 189.6 57.8) (width 0.2) (layer "F.Cu") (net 1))
 (segment (start 163.8 49) (end 185.4 49) (width 0.2) (layer "F.Cu") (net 10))
 (segment (start 192.525 49) (end 195.78 45.745) (width 0.2) (layer "F.Cu") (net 10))
 (segment (start 158.115 35.56) (end 158.115 43.315) (width 0.2) (layer "F.Cu") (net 10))
 (segment (start 158.115 43.315) (end 163.8 49) (width 0.2) (layer "F.Cu") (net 10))
 (segment (start 191 49) (end 192.525 49) (width 0.2) (layer "F.Cu") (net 10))
 (via (at 191 49) (size 0.6) (drill 0.3) (layers "F.Cu" "B.Cu") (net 10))
 (via (at 185.4 49) (size 0.6) (drill 0.3) (layers "F.Cu" "B.Cu") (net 10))
 (segment (start 185.4 49) (end 191 49) (width 0.2) (layer "B.Cu") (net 10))
 (segment (start 186.4 50) (end 193.195 43.205) (width 0.2) (layer "F.Cu") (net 8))
 (segment (start 185.8 50) (end 186.4 50) (width 0.2) (layer "F.Cu") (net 8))
 (segment (start 158.525 54.2) (end 173.4 54.2) (width 0.2) (layer "F.Cu") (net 8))
 (segment (start 193.195 43.205) (end 195.78 43.205) (width 0.2) (layer "F.Cu") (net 8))
 (segment (start 158.115 54.61) (end 158.525 54.2) (width 0.2) (layer "F.Cu") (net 8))
 (via (at 185.8 50) (size 0.6) (drill 0.3) (layers "F.Cu" "B.Cu") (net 8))
 (via (at 173.4 54.2) (size 0.6) (drill 0.3) (layers "F.Cu" "B.Cu") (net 8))
 (segment (start 173.4 54.2) (end 177.6 50) (width 0.2) (layer "B.Cu") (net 8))
 (segment (start 177.6 50) (end 185.8 50) (width 0.2) (layer "B.Cu") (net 8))
 (segment (start 177.165 35.56) (end 190.675 35.56) (width 0.2) (layer "F.Cu") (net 2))
 (segment (start 190.675 35.56) (end 195.78 40.665) (width 0.2) (layer "F.Cu") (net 2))
 (segment (start 177.165 54.61) (end 188.99 54.61) (width 0.2) (layer "B.Cu") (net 9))
 (segment (start 188.99 54.61) (end 192.4 51.2) (width 0.2) (layer "B.Cu") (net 9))
 (segment (start 192.4 40.42737) (end 194.70237 38.125) (width 0.2) (layer "B.Cu") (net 9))
 (segment (start 192.4 51.2) (end 192.4 40.42737) (width 0.2) (layer "B.Cu") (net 9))
 (segment (start 194.70237 38.125) (end 195.78 38.125) (width 0.2) (layer "B.Cu") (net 9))
 (segment (start 139.065 35.56) (end 140.425 34.2) (width 0.2) (layer "F.Cu") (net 7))
 (segment (start 191 31.2) (end 191.6 31.8) (width 0.2) (layer "F.Cu") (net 7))
 (segment (start 191.6 31.8) (end 197.2 31.8) (width 0.2) (layer "F.Cu") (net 7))
 (segment (start 197.2 31.8) (end 197.2 31.6) (width 0.2) (layer "F.Cu") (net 7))
 (segment (start 140.425 34.2) (end 141.2 34.2) (width 0.2) (layer "F.Cu") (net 7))
 (via (at 197.2 31.8) (size 0.6) (drill 0.3) (layers "F.Cu" "B.Cu") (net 7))
 (via (at 191 31.2) (size 0.6) (drill 0.3) (layers "F.Cu" "B.Cu") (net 7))
 (via (at 141.2 34.2) (size 0.6) (drill 0.3) (layers "F.Cu" "B.Cu") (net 7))
 (segment (start 209.6 41.785) (end 211.02 43.205) (width 0.2) (layer "B.Cu") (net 7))
 (segment (start 144.2 31.2) (end 191 31.2) (width 0.2) (layer "B.Cu") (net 7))
 (segment (start 209 28.6) (end 209.6 29.2) (width 0.2) (layer "B.Cu") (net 7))
 (segment (start 197.2 31.8) (end 197.2 28.6) (width 0.2) (layer "B.Cu") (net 7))
 (segment (start 197.2 28.6) (end 209 28.6) (width 0.2) (layer "B.Cu") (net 7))
 (segment (start 141.2 34.2) (end 144.2 31.2) (width 0.2) (layer "B.Cu") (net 7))
 (segment (start 209.6 29.2) (end 209.6 41.785) (width 0.2) (layer "B.Cu") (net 7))
 (segment (start 211.6 65.2) (end 212 64.8) (width 0.2) (layer "F.Cu") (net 3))
 (segment (start 212 64.8) (end 212 46.725) (width 0.2) (layer "F.Cu") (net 3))
 (segment (start 135.4 55.2) (end 135.4 64.2) (width 0.2) (layer "F.Cu") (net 3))
 (segment (start 136.4 65.2) (end 211.6 65.2) (width 0.2) (layer "F.Cu") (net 3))
 (segment (start 212 46.725) (end 211.02 45.745) (width 0.2) (layer "F.Cu") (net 3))
 (segment (start 135.99 54.61) (end 135.4 55.2) (width 0.2) (layer "F.Cu") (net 3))
 (segment (start 139.065 54.61) (end 135.99 54.61) (width 0.2) (layer "F.Cu") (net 3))
 (segment (start 135.4 64.2) (end 136.4 65.2) (width 0.2) (layer "F.Cu") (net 3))
 (segment (start 203.6 55.6) (end 209.8 49.4) (width 0.2) (layer "F.Cu") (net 4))
 (segment (start 209.8 34.265) (end 211.02 33.045) (width 0.2) (layer "F.Cu") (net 4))
 (segment (start 209.8 49.4) (end 209.8 34.265) (width 0.2) (layer "F.Cu") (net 4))
 (segment (start 195.7 55.6) (end 203.6 55.6) (width 0.2) (layer "F.Cu") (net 4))
 (segment (start 212.6 47.007) (end 212.6 42.245) (width 0.2) (layer "F.Cu") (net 5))
 (segment (start 207.6 60.6) (end 207.8 60.4) (width 0.2) (layer "F.Cu") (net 5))
 (segment (start 212.6 42.245) (end 211.02 40.665) (width 0.2) (layer "F.Cu") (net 5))
 (segment (start 195.7 60.6) (end 207.6 60.6) (width 0.2) (layer "F.Cu") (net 5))
 (via (at 212.6 47.007) (size 0.6) (drill 0.3) (layers "F.Cu" "B.Cu") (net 5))
 (via (at 207.8 60.4) (size 0.6) (drill 0.3) (layers "F.Cu" "B.Cu") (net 5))
 (segment (start 211.4 50.8) (end 212.6 49.6) (width 0.2) (layer "B.Cu") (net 5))
 (segment (start 212.6 49.6) (end 212.6 47.007) (width 0.2) (layer "B.Cu") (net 5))
 (segment (start 207.8 54.4) (end 211.4 50.8) (width 0.2) (layer "B.Cu") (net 5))
 (segment (start 207.8 60.4) (end 207.8 54.4) (width 0.2) (layer "B.Cu") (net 5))
 (segment (start 213.2 49) (end 213.2 40.305) (width 0.2) (layer "F.Cu") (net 6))
 (segment (start 213.2 40.305) (end 211.02 38.125) (width 0.2) (layer "F.Cu") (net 6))
 (segment (start 210.2 55.6) (end 210.2 53.2) (width 0.2) (layer "F.Cu") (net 6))
 (via (at 213.2 49) (size 0.6) (drill 0.3) (layers "F.Cu" "B.Cu") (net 6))
 (via (at 210.2 53.2) (size 0.6) (drill 0.3) (layers "F.Cu" "B.Cu") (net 6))
 (segment (start 210.2 53.2) (end 210.4 53.2) (width 0.2) (layer "B.Cu") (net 6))
 (segment (start 210.4 53.2) (end 213.2 50.4) (width 0.2) (layer "B.Cu") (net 6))
 (segment (start 213.2 50.4) (end 213.2 49) (width 0.2) (layer "B.Cu") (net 6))
 (segment (start 209.4 32.125) (end 209.4 40.6) (width 0.2) (layer "F.Cu") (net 11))
 (segment (start 209.4 41.133133) (end 209 41.533133) (width 0.2) (layer "F.Cu") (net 11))
 (segment (start 199.1 44.3) (end 201 44.3) (width 0.2) (layer "F.Cu") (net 11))
 (segment (start 211.02 30.505) (end 209.4 32.125) (width 0.2) (layer "F.Cu") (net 11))
 (segment (start 199 44.4) (end 199.1 44.3) (width 0.2) (layer "F.Cu") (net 11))
 (segment (start 209.4 40.6) (end 209.4 41.133133) (width 0.2) (layer "F.Cu") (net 11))
 (via (at 209 41.533133) (size 0.6) (drill 0.3) (layers "F.Cu" "B.Cu") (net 11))
 (via (at 199 44.4) (size 0.6) (drill 0.3) (layers "F.Cu" "B.Cu") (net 11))
 (segment (start 209 41.533133) (end 209 47.2) (width 0.2) (layer "B.Cu") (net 11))
 (segment (start 198.4 47.4) (end 198.4 45) (width 0.2) (layer "B.Cu") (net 11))
 (segment (start 209 47.2) (end 208.6 47.6) (width 0.2) (layer "B.Cu") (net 11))
 (segment (start 208.6 47.6) (end 206.4 47.6) (width 0.2) (layer "B.Cu") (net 11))
 (segment (start 198.6 47.6) (end 198.4 47.4) (width 0.2) (layer "B.Cu") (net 11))
 (segment (start 206.4 47.6) (end 198.6 47.6) (width 0.2) (layer "B.Cu") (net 11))
 (segment (start 198.4 45) (end 199 44.4) (width 0.2) (layer "B.Cu") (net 11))
 (segment (start 201.2 36) (end 201.2 37.41) (width 0.2) (layer "F.Cu") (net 17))
 (segment (start 206.2 45.8) (end 207.8 45.8) (width 0.2) (layer "F.Cu") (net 17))
 (segment (start 201.2 37.41) (end 201.0125 37.5975) (width 0.2) (layer "F.Cu") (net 17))
 (segment (start 207.8 45.8) (end 208.2 45.4) (width 0.2) (layer "F.Cu") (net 17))
 (via (at 201.2 36) (size 0.6) (drill 0.3) (layers "F.Cu" "B.Cu") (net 17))
 (via (at 208.2 45.4) (size 0.6) (drill 0.3) (layers "F.Cu" "B.Cu") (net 17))
 (segment (start 207.6 44.8) (end 207.6 36) (width 0.2) (layer "B.Cu") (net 17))
 (segment (start 208.2 45.4) (end 207.6 44.8) (width 0.2) (layer "B.Cu") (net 17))
 (segment (start 207.6 36) (end 201.2 36) (width 0.2) (layer "B.Cu") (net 17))
 (segment (start 199.2 31.6) (end 201 31.6) (width 0.2) (layer "F.Cu") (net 16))
 (segment (start 199.2 40.8) (end 199 40.6) (width 0.2) (layer "F.Cu") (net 16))
 (segment (start 206.2125 40.1875) (end 205.6 40.8) (width 0.2) (layer "F.Cu") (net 16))
 (segment (start 205.6 40.8) (end 199.2 40.8) (width 0.2) (layer "F.Cu") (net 16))
 (segment (start 206.2125 39.0975) (end 206.2125 40.1875) (width 0.2) (layer "F.Cu") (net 16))
 (via (at 199.2 31.6) (size 0.6) (drill 0.3) (layers "F.Cu" "B.Cu") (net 16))
 (via (at 199 40.6) (size 0.6) (drill 0.3) (layers "F.Cu" "B.Cu") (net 16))
 (segment (start 199 31.8) (end 199.2 31.6) (width 0.2) (layer "B.Cu") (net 16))
 (segment (start 199 40.6) (end 199 31.8) (width 0.2) (layer "B.Cu") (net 16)))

